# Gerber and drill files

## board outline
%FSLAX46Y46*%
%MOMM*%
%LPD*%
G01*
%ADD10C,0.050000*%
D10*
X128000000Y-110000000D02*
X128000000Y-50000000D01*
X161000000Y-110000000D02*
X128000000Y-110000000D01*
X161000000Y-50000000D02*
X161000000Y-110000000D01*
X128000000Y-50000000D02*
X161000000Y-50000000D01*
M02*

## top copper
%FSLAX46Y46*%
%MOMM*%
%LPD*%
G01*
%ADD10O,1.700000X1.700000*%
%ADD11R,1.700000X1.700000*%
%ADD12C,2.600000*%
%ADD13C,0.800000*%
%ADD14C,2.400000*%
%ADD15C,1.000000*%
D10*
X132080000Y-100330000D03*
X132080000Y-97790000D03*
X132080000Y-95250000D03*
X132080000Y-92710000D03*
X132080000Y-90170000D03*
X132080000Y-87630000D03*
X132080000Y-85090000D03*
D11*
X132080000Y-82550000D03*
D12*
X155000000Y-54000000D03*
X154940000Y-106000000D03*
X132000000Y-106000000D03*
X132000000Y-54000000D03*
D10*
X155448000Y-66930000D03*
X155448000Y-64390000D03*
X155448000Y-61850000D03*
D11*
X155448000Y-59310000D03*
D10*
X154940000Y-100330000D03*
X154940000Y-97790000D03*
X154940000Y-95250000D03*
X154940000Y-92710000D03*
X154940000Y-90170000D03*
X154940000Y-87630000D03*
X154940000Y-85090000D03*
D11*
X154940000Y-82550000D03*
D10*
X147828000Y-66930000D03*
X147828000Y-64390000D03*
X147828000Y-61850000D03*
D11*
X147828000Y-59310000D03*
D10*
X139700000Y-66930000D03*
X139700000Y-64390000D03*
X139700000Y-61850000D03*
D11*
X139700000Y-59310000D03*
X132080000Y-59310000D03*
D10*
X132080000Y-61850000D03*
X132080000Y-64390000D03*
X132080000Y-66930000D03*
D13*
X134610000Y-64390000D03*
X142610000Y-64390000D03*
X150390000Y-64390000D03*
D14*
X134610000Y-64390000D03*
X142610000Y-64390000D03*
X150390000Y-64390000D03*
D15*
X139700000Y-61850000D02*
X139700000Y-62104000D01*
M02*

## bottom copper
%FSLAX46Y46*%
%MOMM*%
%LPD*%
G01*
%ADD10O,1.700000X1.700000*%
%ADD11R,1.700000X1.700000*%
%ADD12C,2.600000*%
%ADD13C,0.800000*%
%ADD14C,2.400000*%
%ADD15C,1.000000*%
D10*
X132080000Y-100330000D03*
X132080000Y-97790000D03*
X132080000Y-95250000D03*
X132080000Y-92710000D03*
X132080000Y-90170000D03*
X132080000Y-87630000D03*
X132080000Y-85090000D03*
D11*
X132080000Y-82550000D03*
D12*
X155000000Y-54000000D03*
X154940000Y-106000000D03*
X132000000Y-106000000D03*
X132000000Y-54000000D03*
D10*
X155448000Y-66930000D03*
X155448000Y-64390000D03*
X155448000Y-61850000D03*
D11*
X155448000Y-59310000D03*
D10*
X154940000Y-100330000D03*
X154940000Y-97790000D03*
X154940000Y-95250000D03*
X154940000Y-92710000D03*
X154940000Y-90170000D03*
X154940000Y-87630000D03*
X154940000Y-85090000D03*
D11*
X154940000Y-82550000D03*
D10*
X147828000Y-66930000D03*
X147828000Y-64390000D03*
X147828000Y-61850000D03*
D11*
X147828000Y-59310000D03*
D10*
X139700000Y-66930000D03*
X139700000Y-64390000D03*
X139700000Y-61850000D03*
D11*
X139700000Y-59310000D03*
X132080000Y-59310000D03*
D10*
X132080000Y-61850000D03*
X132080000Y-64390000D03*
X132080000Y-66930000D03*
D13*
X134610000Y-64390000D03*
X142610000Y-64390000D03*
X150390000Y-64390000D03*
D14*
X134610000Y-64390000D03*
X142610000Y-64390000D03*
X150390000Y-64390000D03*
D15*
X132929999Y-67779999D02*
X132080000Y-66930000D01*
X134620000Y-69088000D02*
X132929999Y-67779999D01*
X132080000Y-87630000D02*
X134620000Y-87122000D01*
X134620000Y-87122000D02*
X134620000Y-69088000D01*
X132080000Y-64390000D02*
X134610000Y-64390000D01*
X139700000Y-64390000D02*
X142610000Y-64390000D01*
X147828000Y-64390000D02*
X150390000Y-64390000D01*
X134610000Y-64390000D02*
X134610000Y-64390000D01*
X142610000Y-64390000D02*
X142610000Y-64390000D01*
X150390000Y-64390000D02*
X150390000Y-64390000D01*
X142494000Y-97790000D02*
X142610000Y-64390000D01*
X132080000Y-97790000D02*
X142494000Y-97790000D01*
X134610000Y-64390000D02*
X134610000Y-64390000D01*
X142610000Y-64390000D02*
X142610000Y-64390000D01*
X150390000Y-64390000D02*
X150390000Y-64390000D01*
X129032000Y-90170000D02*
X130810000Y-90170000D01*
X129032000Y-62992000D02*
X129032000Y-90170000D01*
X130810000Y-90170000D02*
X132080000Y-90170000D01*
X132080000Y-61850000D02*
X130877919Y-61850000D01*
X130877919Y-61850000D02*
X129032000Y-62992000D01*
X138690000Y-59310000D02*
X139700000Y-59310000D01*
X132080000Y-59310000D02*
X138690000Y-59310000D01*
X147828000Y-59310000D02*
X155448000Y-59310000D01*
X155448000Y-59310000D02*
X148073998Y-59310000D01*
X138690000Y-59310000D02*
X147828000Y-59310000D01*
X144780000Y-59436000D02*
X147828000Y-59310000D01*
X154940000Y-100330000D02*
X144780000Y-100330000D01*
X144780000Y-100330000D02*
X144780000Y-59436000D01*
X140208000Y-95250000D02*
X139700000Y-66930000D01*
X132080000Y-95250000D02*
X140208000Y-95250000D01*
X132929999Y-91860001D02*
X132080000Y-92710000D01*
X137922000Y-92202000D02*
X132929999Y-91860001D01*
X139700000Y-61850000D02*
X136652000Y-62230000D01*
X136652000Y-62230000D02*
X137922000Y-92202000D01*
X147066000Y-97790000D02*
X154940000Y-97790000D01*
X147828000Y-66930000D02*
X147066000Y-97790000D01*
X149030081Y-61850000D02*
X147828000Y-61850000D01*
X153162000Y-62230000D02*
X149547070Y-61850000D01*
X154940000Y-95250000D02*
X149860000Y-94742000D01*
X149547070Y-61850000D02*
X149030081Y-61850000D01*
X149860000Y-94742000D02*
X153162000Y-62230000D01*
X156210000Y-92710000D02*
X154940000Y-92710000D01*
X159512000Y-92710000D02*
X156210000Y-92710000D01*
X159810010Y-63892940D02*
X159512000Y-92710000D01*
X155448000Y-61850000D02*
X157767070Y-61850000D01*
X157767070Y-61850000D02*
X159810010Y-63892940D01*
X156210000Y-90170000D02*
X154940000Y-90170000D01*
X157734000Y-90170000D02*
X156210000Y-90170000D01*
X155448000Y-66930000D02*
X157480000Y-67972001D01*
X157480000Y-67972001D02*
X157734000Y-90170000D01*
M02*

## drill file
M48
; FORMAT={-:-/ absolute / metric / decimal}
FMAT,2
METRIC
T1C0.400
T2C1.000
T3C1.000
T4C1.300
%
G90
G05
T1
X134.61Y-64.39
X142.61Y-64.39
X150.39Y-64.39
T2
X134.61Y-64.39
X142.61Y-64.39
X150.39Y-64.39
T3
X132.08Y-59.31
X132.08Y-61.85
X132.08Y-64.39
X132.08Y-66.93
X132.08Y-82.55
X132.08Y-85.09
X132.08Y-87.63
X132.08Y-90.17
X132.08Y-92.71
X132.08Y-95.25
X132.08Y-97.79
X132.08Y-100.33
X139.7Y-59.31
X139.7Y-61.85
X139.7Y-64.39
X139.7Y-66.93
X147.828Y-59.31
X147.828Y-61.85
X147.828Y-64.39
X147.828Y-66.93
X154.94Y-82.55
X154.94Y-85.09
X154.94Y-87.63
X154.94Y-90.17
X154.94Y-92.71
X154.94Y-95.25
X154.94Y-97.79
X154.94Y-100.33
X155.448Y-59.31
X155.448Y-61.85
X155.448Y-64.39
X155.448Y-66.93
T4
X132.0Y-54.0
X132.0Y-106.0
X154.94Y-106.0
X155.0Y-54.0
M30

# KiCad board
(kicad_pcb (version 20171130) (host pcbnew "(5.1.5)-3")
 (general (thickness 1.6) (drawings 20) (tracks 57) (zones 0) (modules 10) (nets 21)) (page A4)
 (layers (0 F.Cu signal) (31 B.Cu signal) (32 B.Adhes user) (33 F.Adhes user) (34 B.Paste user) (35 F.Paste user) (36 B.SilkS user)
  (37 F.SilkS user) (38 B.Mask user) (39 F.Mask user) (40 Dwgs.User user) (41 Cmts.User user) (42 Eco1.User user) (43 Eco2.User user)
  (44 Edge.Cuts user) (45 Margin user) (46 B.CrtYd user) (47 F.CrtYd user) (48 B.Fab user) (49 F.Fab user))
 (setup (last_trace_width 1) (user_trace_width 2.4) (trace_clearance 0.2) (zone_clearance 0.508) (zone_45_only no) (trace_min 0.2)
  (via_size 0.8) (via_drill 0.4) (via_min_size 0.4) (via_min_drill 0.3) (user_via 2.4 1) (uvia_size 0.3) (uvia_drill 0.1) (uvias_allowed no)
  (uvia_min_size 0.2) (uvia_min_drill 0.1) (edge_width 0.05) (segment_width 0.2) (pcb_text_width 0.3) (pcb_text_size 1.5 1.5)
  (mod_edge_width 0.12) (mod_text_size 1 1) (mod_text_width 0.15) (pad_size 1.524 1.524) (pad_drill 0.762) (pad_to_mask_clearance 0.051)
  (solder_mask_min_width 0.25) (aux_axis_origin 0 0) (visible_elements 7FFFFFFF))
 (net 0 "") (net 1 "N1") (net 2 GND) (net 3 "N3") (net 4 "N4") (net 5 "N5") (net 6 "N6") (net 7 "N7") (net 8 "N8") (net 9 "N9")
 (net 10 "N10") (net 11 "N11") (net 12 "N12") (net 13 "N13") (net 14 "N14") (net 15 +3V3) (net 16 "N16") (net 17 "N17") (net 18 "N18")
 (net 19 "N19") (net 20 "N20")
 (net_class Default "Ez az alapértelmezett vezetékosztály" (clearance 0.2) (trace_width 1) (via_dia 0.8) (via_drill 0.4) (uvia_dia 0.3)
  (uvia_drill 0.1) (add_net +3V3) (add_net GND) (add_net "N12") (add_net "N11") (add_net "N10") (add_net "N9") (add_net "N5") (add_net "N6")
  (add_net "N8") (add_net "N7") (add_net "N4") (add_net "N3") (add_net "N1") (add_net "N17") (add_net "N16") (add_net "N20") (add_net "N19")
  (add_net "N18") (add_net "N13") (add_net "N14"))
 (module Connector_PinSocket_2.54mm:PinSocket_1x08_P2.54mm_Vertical (layer F.Cu) (at 132.08 82.55)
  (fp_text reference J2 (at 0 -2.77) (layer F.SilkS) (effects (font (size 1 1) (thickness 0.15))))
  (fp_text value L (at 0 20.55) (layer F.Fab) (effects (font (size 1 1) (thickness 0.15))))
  (pad 8 thru_hole oval (at 0 17.78) (size 1.7 1.7) (drill 1) (layers *.Cu *.Mask) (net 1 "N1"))
  (pad 7 thru_hole oval (at 0 15.24) (size 1.7 1.7) (drill 1) (layers *.Cu *.Mask) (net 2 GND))
  (pad 6 thru_hole oval (at 0 12.7) (size 1.7 1.7) (drill 1) (layers *.Cu *.Mask) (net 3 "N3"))
  (pad 5 thru_hole oval (at 0 10.16) (size 1.7 1.7) (drill 1) (layers *.Cu *.Mask) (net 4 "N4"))
  (pad 4 thru_hole oval (at 0 7.62) (size 1.7 1.7) (drill 1) (layers *.Cu *.Mask) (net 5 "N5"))
  (pad 3 thru_hole oval (at 0 5.08) (size 1.7 1.7) (drill 1) (layers *.Cu *.Mask) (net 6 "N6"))
  (pad 2 thru_hole oval (at 0 2.54) (size 1.7 1.7) (drill 1) (layers *.Cu *.Mask) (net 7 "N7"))
  (pad 1 thru_hole rect (at 0 0) (size 1.7 1.7) (drill 1) (layers *.Cu *.Mask) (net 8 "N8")))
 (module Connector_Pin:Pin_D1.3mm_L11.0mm (layer F.Cu) (at 155 54)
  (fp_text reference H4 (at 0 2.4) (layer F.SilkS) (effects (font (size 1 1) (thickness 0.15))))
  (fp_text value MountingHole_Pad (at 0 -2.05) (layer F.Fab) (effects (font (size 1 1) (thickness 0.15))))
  (pad 1 thru_hole circle (at 0 0) (size 2.6 2.6) (drill 1.3) (layers *.Cu *.Mask) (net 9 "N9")))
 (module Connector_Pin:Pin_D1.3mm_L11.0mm (layer F.Cu) (at 154.94 106)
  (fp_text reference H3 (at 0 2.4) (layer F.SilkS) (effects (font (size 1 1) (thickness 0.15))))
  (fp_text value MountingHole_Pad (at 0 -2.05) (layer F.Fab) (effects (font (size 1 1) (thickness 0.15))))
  (pad 1 thru_hole circle (at 0 0) (size 2.6 2.6) (drill 1.3) (layers *.Cu *.Mask) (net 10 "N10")))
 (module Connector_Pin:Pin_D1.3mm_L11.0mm (layer F.Cu) (at 132 106)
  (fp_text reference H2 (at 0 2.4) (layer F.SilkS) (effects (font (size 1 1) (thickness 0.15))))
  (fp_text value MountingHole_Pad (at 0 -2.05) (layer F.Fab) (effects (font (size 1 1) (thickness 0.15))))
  (pad 1 thru_hole circle (at 0 0) (size 2.6 2.6) (drill 1.3) (layers *.Cu *.Mask) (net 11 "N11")))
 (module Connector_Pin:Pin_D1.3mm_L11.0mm (layer F.Cu) (at 132 54)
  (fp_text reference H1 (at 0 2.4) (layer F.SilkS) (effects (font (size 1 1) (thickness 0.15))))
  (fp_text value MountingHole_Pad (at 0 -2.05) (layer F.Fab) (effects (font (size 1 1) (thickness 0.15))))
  (pad 1 thru_hole circle (at 0 0) (size 2.6 2.6) (drill 1.3) (layers *.Cu *.Mask) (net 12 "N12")))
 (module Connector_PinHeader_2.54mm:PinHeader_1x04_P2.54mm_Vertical (layer F.Cu) (at 155.448 59.31)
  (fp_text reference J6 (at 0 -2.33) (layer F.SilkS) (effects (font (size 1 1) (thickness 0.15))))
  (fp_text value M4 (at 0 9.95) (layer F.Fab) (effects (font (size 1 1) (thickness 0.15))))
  (pad 4 thru_hole oval (at 0 7.62) (size 1.7 1.7) (drill 1) (layers *.Cu *.Mask) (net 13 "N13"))
  (pad 3 thru_hole oval (at 0 5.08) (size 1.7 1.7) (drill 1) (layers *.Cu *.Mask) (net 2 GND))
  (pad 2 thru_hole oval (at 0 2.54) (size 1.7 1.7) (drill 1) (layers *.Cu *.Mask) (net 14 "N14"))
  (pad 1 thru_hole rect (at 0 0) (size 1.7 1.7) (drill 1) (layers *.Cu *.Mask) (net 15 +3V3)))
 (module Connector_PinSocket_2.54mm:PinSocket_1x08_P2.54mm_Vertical (layer F.Cu) (at 154.94 82.55)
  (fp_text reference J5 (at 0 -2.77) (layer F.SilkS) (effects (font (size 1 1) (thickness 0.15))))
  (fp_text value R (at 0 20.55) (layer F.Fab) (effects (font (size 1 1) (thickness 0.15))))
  (pad 8 thru_hole oval (at 0 17.78) (size 1.7 1.7) (drill 1) (layers *.Cu *.Mask) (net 15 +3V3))
  (pad 7 thru_hole oval (at 0 15.24) (size 1.7 1.7) (drill 1) (layers *.Cu *.Mask) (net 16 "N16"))
  (pad 6 thru_hole oval (at 0 12.7) (size 1.7 1.7) (drill 1) (layers *.Cu *.Mask) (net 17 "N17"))
  (pad 5 thru_hole oval (at 0 10.16) (size 1.7 1.7) (drill 1) (layers *.Cu *.Mask) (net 14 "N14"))
  (pad 4 thru_hole oval (at 0 7.62) (size 1.7 1.7) (drill 1) (layers *.Cu *.Mask) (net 13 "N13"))
  (pad 3 thru_hole oval (at 0 5.08) (size 1.7 1.7) (drill 1) (layers *.Cu *.Mask) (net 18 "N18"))
  (pad 2 thru_hole oval (at 0 2.54) (size 1.7 1.7) (drill 1) (layers *.Cu *.Mask) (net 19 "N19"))
  (pad 1 thru_hole rect (at 0 0) (size 1.7 1.7) (drill 1) (layers *.Cu *.Mask) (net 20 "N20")))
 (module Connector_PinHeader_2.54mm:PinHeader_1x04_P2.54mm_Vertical (layer F.Cu) (at 147.828 59.31)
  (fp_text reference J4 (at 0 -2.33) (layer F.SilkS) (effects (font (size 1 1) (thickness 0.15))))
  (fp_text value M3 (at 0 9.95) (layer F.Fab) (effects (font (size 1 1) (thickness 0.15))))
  (pad 4 thru_hole oval (at 0 7.62) (size 1.7 1.7) (drill 1) (layers *.Cu *.Mask) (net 16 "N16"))
  (pad 3 thru_hole oval (at 0 5.08) (size 1.7 1.7) (drill 1) (layers *.Cu *.Mask) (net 2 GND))
  (pad 2 thru_hole oval (at 0 2.54) (size 1.7 1.7) (drill 1) (layers *.Cu *.Mask) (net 17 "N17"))
  (pad 1 thru_hole rect (at 0 0) (size 1.7 1.7) (drill 1) (layers *.Cu *.Mask) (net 15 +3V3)))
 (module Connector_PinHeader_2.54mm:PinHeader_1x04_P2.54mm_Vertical (layer F.Cu) (at 139.7 59.31)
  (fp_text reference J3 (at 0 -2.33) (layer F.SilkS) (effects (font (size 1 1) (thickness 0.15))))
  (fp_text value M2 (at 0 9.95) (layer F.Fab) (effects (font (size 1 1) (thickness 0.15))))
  (pad 4 thru_hole oval (at 0 7.62) (size 1.7 1.7) (drill 1) (layers *.Cu *.Mask) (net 3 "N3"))
  (pad 3 thru_hole oval (at 0 5.08) (size 1.7 1.7) (drill 1) (layers *.Cu *.Mask) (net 2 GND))
  (pad 2 thru_hole oval (at 0 2.54) (size 1.7 1.7) (drill 1) (layers *.Cu *.Mask) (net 4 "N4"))
  (pad 1 thru_hole rect (at 0 0) (size 1.7 1.7) (drill 1) (layers *.Cu *.Mask) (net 15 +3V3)))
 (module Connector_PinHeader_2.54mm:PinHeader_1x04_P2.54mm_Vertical (layer F.Cu) (at 132.08 59.31)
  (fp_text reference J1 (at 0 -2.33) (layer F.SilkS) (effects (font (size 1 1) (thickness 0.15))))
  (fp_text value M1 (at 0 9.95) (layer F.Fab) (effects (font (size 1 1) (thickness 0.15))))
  (pad 1 thru_hole rect (at 0 0) (size 1.7 1.7) (drill 1) (layers *.Cu *.Mask) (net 15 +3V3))
  (pad 2 thru_hole oval (at 0 2.54) (size 1.7 1.7) (drill 1) (layers *.Cu *.Mask) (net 5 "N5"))
  (pad 3 thru_hole oval (at 0 5.08) (size 1.7 1.7) (drill 1) (layers *.Cu *.Mask) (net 2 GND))
  (pad 4 thru_hole oval (at 0 7.62) (size 1.7 1.7) (drill 1) (layers *.Cu *.Mask) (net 6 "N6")))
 (gr_line (start 128 110) (end 128 50) (layer Edge.Cuts) (width 0.05))
 (gr_line (start 161 110) (end 128 110) (layer Edge.Cuts) (width 0.05))
 (gr_line (start 161 50) (end 161 110) (layer Edge.Cuts) (width 0.05))
 (gr_line (start 128 50) (end 161 50) (layer Edge.Cuts) (width 0.05))
 (segment (start 132.929999 67.779999) (end 132.08 66.93) (width 1) (layer B.Cu) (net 6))
 (segment (start 134.62 69.088) (end 132.929999 67.779999) (width 1) (layer B.Cu) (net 6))
 (segment (start 132.08 87.63) (end 134.62 87.122) (width 1) (layer B.Cu) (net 6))
 (segment (start 134.62 87.122) (end 134.62 69.088) (width 1) (layer B.Cu) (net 6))
 (segment (start 132.08 64.39) (end 134.61 64.39) (width 1) (layer B.Cu) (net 2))
 (segment (start 139.7 64.39) (end 142.61 64.39) (width 1) (layer B.Cu) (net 2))
 (segment (start 147.828 64.39) (end 150.39 64.39) (width 1) (layer B.Cu) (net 2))
 (segment (start 134.61 64.39) (end 134.61 64.39) (width 1) (layer B.Cu) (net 2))
 (via (at 134.61 64.39) (size 0.8) (drill 0.4) (layers F.Cu B.Cu) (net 2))
 (segment (start 142.61 64.39) (end 142.61 64.39) (width 1) (layer B.Cu) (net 2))
 (via (at 142.61 64.39) (size 0.8) (drill 0.4) (layers F.Cu B.Cu) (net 2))
 (segment (start 150.39 64.39) (end 150.39 64.39) (width 1) (layer B.Cu) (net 2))
 (via (at 150.39 64.39) (size 0.8) (drill 0.4) (layers F.Cu B.Cu) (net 2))
 (segment (start 142.494 97.79) (end 142.61 64.39) (width 1) (layer B.Cu) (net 2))
 (segment (start 132.08 97.79) (end 142.494 97.79) (width 1) (layer B.Cu) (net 2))
 (segment (start 134.61 64.39) (end 134.61 64.39) (width 1) (layer B.Cu) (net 2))
 (via (at 134.61 64.39) (size 2.4) (drill 1) (layers F.Cu B.Cu) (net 2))
 (segment (start 142.61 64.39) (end 142.61 64.39) (width 1) (layer B.Cu) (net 2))
 (via (at 142.61 64.39) (size 2.4) (drill 1) (layers F.Cu B.Cu) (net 2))
 (segment (start 150.39 64.39) (end 150.39 64.39) (width 1) (layer B.Cu) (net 2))
 (via (at 150.39 64.39) (size 2.4) (drill 1) (layers F.Cu B.Cu) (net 2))
 (segment (start 129.032 90.17) (end 130.81 90.17) (width 1) (layer B.Cu) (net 5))
 (segment (start 129.032 62.992) (end 129.032 90.17) (width 1) (layer B.Cu) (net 5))
 (segment (start 130.81 90.17) (end 132.08 90.17) (width 1) (layer B.Cu) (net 5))
 (segment (start 132.08 61.85) (end 130.877919 61.85) (width 1) (layer B.Cu) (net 5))
 (segment (start 130.877919 61.85) (end 129.032 62.992) (width 1) (layer B.Cu) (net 5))
 (segment (start 138.69 59.31) (end 139.7 59.31) (width 1) (layer B.Cu) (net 15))
 (segment (start 132.08 59.31) (end 138.69 59.31) (width 1) (layer B.Cu) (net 15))
 (segment (start 147.828 59.31) (end 155.448 59.31) (width 1) (layer B.Cu) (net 15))
 (segment (start 155.448 59.31) (end 148.073998 59.31) (width 1) (layer B.Cu) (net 15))
 (segment (start 138.69 59.31) (end 147.828 59.31) (width 1) (layer B.Cu) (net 15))
 (segment (start 144.78 59.436) (end 147.828 59.31) (width 1) (layer B.Cu) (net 15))
 (segment (start 154.94 100.33) (end 144.78 100.33) (width 1) (layer B.Cu) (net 15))
 (segment (start 144.78 100.33) (end 144.78 59.436) (width 1) (layer B.Cu) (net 15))
 (segment (start 140.208 95.25) (end 139.7 66.93) (width 1) (layer B.Cu) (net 3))
 (segment (start 132.08 95.25) (end 140.208 95.25) (width 1) (layer B.Cu) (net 3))
 (segment (start 139.7 61.85) (end 139.7 62.104) (width 1) (layer F.Cu) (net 4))
 (segment (start 132.929999 91.860001) (end 132.08 92.71) (width 1) (layer B.Cu) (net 4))
 (segment (start 137.922 92.202) (end 132.929999 91.860001) (width 1) (layer B.Cu) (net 4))
 (segment (start 139.7 61.85) (end 136.652 62.23) (width 1) (layer B.Cu) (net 4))
 (segment (start 136.652 62.23) (end 137.922 92.202) (width 1) (layer B.Cu) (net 4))
 (segment (start 147.066 97.79) (end 154.94 97.79) (width 1) (layer B.Cu) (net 16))
 (segment (start 147.828 66.93) (end 147.066 97.79) (width 1) (layer B.Cu) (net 16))
 (segment (start 149.030081 61.85) (end 147.828 61.85) (width 1) (layer B.Cu) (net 17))
 (segment (start 153.162 62.23) (end 149.54707 61.85) (width 1) (layer B.Cu) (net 17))
 (segment (start 154.94 95.25) (end 149.86 94.742) (width 1) (layer B.Cu) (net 17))
 (segment (start 149.54707 61.85) (end 149.030081 61.85) (width 1) (layer B.Cu) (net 17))
 (segment (start 149.86 94.742) (end 153.162 62.23) (width 1) (layer B.Cu) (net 17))
 (segment (start 156.21 92.71) (end 154.94 92.71) (width 1) (layer B.Cu) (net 14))
 (segment (start 159.512 92.71) (end 156.21 92.71) (width 1) (layer B.Cu) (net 14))
 (segment (start 159.81001 63.89294) (end 159.512 92.71) (width 1) (layer B.Cu) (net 14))
 (segment (start 155.448 61.85) (end 157.76707 61.85) (width 1) (layer B.Cu) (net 14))
 (segment (start 157.76707 61.85) (end 159.81001 63.89294) (width 1) (layer B.Cu) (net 14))
 (segment (start 156.21 90.17) (end 154.94 90.17) (width 1) (layer B.Cu) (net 13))
 (segment (start 157.734 90.17) (end 156.21 90.17) (width 1) (layer B.Cu) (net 13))
 (segment (start 155.448 66.93) (end 157.48 67.972001) (width 1) (layer B.Cu) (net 13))
 (segment (start 157.48 67.972001) (end 157.734 90.17) (width 1) (layer B.Cu) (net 13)))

